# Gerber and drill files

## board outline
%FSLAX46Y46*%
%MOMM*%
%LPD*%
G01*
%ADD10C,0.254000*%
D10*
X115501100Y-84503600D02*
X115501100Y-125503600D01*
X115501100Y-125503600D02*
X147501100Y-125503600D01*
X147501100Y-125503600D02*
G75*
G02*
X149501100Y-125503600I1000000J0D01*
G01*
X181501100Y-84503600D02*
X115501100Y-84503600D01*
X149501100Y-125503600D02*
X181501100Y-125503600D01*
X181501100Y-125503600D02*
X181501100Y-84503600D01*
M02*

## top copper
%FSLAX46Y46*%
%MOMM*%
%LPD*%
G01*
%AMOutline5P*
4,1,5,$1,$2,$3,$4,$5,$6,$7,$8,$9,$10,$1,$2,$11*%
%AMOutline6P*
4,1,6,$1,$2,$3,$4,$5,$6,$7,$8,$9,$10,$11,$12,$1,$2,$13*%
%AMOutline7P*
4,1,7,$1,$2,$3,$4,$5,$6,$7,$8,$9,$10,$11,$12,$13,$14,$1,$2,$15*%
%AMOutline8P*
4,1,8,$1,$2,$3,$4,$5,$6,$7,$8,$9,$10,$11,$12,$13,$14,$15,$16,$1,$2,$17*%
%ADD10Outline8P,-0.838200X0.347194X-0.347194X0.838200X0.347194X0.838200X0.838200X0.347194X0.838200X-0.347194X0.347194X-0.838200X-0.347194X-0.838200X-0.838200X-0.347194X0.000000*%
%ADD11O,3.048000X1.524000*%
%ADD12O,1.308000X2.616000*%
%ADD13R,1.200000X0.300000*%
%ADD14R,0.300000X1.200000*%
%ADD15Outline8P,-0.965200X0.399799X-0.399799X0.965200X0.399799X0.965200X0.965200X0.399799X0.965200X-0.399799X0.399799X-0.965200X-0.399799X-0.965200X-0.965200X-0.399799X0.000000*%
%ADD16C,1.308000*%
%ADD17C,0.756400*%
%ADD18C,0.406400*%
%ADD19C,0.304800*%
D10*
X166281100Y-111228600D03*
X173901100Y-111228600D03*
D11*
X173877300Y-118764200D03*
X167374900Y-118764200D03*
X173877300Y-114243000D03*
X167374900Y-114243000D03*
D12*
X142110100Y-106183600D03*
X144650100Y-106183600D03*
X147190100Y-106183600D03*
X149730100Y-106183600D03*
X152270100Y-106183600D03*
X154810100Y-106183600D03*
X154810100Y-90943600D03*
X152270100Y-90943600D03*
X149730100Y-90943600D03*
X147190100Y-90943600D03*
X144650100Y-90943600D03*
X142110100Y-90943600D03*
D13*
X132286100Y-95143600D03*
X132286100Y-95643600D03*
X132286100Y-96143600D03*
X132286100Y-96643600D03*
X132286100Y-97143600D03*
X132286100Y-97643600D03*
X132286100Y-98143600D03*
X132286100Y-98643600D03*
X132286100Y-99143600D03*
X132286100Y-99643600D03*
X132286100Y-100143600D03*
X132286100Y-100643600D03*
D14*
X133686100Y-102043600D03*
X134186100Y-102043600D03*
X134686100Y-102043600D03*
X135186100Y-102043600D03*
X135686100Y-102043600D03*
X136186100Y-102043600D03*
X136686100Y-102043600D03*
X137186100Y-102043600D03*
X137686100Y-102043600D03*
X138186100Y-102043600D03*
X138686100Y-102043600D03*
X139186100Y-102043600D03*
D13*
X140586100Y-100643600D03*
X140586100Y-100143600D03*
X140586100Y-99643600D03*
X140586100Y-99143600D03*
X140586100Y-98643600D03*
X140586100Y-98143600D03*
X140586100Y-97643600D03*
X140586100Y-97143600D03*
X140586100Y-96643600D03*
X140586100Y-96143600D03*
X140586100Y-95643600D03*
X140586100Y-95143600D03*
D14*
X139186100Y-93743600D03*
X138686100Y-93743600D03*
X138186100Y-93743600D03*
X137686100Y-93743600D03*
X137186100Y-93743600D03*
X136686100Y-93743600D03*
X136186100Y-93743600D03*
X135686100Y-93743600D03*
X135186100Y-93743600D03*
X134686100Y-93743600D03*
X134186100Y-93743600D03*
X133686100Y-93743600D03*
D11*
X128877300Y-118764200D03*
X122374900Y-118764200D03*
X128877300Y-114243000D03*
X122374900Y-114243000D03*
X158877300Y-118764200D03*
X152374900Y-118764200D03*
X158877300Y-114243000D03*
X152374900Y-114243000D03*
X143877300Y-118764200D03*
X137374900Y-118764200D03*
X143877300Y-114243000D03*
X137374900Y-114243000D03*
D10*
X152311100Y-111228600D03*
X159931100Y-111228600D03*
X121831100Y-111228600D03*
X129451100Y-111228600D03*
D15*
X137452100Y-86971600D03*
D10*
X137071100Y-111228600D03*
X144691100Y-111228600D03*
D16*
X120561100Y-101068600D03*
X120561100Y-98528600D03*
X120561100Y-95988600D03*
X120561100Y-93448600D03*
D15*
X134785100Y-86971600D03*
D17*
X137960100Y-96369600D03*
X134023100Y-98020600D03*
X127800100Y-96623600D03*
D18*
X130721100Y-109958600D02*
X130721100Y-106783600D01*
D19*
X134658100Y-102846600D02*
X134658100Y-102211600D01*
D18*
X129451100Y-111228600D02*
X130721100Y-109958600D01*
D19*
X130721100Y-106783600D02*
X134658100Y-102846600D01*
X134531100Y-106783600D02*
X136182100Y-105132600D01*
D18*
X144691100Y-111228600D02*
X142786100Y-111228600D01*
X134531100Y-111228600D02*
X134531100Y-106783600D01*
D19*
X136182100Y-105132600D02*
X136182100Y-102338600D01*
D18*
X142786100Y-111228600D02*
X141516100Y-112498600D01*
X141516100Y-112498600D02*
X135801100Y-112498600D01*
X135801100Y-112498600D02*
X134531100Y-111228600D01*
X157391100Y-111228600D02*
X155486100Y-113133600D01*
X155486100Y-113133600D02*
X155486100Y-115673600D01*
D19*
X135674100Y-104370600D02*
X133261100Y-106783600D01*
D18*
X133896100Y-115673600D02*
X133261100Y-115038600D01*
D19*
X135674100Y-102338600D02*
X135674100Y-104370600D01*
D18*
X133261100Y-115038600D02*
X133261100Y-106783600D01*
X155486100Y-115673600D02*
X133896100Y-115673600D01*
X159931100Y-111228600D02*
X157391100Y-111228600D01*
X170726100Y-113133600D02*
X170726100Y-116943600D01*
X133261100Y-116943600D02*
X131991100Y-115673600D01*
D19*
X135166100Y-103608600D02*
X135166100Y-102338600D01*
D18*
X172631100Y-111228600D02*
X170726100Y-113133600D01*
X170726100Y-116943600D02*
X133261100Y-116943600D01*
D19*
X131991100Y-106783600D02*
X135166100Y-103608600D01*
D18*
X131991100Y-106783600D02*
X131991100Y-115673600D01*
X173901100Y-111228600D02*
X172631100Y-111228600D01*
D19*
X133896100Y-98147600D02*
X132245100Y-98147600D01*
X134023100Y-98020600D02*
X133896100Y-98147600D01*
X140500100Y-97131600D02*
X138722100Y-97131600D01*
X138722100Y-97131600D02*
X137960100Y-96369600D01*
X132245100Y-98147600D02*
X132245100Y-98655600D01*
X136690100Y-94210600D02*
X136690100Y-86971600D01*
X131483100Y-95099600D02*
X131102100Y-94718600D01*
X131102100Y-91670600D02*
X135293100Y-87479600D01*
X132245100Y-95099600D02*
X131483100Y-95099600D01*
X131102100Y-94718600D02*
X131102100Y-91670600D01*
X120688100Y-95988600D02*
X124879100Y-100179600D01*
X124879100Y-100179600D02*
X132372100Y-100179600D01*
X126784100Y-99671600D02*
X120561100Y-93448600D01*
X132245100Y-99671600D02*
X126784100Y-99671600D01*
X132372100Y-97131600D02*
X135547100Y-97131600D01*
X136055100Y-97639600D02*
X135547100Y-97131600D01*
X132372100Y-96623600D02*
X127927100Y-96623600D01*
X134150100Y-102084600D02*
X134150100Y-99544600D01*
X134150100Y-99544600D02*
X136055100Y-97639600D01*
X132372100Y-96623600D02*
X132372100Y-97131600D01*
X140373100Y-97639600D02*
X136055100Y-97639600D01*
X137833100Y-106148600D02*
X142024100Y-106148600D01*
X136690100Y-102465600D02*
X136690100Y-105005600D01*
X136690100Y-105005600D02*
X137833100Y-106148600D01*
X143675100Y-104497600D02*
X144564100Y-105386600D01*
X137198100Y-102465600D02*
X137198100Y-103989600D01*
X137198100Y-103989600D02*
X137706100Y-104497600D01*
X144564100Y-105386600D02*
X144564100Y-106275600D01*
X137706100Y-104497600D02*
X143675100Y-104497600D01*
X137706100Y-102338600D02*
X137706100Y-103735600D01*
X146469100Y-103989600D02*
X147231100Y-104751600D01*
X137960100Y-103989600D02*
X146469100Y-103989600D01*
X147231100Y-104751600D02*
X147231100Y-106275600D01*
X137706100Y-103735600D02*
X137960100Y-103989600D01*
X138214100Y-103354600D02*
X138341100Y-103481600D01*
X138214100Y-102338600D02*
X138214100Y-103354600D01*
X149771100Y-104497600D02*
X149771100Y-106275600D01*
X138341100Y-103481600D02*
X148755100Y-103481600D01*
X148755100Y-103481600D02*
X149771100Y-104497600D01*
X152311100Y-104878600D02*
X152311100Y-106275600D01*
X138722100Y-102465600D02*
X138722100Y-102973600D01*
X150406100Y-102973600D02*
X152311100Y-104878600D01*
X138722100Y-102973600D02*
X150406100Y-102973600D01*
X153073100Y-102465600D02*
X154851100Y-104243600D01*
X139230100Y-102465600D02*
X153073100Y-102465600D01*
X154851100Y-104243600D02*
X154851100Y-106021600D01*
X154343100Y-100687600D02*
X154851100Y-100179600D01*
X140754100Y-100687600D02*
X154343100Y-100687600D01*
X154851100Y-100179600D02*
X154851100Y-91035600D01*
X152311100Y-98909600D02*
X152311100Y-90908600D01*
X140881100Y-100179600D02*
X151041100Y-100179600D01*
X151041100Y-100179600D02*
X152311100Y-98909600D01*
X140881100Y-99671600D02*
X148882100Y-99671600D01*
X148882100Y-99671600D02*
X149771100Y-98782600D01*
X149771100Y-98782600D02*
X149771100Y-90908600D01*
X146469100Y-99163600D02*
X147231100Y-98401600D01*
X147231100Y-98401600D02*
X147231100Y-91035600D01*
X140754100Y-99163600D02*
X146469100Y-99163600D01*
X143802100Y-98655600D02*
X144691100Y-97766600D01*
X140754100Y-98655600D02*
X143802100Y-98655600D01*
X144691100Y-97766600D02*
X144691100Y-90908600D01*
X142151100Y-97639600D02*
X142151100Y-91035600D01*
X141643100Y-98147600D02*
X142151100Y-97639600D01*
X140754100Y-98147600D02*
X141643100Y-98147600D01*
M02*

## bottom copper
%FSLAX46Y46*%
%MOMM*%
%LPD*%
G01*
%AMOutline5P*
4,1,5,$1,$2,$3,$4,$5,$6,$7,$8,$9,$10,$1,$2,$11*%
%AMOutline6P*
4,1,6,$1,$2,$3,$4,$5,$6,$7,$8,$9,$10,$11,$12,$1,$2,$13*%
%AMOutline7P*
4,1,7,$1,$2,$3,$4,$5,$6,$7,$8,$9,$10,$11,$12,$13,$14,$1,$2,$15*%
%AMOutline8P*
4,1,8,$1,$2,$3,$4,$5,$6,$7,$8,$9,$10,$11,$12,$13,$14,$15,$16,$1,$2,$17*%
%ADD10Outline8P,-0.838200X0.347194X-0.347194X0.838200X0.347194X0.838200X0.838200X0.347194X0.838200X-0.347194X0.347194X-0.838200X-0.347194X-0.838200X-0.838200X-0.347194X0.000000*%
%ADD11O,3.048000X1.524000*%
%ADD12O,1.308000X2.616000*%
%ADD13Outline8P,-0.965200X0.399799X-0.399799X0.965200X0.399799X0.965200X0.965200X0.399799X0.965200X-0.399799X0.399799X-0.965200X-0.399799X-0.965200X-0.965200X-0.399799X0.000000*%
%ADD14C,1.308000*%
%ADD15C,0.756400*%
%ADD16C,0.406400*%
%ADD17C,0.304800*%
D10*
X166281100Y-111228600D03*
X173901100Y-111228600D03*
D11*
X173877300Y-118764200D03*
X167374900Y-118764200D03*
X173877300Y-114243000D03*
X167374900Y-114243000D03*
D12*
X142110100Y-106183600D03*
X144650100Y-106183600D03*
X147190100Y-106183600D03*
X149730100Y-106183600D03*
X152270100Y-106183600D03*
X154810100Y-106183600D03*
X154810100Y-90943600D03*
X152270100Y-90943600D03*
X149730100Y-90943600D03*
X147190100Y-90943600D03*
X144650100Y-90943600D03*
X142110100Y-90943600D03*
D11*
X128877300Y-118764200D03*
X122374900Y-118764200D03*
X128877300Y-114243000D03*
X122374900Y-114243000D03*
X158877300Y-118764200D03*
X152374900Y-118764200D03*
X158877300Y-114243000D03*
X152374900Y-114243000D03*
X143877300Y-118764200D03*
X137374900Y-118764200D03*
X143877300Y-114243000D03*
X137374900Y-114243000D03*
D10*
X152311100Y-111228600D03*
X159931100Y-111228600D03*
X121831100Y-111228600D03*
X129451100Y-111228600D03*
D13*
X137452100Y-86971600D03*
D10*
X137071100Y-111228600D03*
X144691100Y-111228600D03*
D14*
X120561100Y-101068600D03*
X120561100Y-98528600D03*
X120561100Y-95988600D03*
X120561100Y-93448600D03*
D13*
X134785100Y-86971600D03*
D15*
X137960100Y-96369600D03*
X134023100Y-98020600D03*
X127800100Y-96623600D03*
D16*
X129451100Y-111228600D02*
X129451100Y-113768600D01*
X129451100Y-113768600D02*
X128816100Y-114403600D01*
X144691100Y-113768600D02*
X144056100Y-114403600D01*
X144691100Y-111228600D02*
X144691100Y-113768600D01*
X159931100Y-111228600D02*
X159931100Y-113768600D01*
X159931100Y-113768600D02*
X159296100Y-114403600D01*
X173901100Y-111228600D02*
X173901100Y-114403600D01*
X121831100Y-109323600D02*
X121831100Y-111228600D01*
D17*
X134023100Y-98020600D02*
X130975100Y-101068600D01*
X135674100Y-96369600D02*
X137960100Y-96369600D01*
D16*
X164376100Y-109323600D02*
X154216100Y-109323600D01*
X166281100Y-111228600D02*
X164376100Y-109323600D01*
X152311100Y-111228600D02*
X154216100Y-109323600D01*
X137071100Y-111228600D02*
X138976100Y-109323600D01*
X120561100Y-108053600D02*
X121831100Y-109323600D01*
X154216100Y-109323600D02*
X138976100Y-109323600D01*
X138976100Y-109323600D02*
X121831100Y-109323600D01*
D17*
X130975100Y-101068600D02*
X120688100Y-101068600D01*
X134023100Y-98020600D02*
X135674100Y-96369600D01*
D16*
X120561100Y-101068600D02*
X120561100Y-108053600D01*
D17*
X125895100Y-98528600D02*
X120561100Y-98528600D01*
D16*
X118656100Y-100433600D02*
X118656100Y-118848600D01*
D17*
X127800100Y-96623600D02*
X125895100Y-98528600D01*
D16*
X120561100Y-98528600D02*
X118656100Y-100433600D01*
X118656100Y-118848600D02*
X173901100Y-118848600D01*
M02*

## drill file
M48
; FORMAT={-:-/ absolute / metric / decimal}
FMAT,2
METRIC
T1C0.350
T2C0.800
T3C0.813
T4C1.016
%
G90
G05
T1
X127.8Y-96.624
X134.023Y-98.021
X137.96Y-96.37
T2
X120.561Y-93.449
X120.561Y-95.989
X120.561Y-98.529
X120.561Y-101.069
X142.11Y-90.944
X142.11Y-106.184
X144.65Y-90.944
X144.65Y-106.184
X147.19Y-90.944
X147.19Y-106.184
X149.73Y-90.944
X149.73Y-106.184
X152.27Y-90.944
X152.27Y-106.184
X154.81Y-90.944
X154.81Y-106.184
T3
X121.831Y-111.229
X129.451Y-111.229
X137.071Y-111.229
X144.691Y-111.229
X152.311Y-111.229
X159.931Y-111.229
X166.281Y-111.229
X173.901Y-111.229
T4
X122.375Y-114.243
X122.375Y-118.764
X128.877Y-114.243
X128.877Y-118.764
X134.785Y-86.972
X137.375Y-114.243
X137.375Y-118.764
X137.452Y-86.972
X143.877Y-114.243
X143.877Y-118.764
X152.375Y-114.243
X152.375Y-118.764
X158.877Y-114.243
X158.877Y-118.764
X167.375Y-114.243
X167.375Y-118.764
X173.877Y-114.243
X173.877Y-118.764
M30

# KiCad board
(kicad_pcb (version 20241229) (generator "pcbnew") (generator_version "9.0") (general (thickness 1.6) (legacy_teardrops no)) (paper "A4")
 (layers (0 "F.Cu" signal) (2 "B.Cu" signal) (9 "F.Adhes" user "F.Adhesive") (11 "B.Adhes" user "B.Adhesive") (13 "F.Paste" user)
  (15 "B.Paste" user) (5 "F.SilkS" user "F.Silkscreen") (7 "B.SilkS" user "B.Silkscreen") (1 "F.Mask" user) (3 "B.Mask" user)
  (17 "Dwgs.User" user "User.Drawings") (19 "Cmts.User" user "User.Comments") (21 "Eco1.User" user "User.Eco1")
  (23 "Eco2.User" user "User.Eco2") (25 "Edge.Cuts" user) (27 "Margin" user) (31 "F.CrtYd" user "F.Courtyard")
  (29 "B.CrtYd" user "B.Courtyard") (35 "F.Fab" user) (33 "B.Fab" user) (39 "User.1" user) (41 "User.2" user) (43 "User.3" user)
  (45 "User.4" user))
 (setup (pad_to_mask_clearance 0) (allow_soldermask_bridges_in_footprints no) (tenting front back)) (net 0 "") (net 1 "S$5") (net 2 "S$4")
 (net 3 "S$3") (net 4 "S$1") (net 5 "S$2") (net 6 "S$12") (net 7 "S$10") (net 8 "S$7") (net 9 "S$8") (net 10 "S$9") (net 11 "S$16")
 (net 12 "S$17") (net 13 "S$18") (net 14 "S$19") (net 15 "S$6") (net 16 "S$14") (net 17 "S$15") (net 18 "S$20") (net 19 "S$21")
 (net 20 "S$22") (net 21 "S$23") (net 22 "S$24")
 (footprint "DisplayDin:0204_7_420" (layer "F.Cu") (at 170.0911 111.2286)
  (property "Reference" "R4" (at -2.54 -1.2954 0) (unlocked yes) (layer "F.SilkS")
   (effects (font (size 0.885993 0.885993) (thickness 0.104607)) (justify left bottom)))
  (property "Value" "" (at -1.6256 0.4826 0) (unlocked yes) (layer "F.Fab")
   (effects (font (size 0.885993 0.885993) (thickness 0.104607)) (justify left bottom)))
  (pad "1" thru_hole roundrect (at -3.81 0) (size 1.6764 1.6764) (drill 0.8128) (layers "*.Cu" "*.Mask") (remove_unused_layers no)
   (roundrect_rratio 0.25) (chamfer_ratio 0.2928932188) (chamfer top_left top_right bottom_left bottom_right) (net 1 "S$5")
   (solder_mask_margin 0.1016) (thermal_bridge_angle 0))
  (pad "2" thru_hole roundrect (at 3.81 0) (size 1.6764 1.6764) (drill 0.8128) (layers "*.Cu" "*.Mask") (remove_unused_layers no)
   (roundrect_rratio 0.25) (chamfer_ratio 0.2928932188) (chamfer top_left top_right bottom_left bottom_right) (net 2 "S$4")
   (solder_mask_margin 0.1016) (thermal_bridge_angle 0)))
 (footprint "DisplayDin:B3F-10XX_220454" (layer "F.Cu") (at 170.6261 116.5036 180)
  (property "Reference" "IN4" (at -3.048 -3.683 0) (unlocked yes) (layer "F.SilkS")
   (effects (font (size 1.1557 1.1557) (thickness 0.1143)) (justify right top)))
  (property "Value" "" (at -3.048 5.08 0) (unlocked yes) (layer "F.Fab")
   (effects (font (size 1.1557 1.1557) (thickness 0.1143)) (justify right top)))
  (pad "1" thru_hole oval (at -3.2512 -2.2606 180) (size 3.048 1.524) (drill 1.016) (layers "*.Cu" "*.Mask") (remove_unused_layers no)
   (solder_mask_margin 0.1016) (thermal_bridge_angle 0))
  (pad "2" thru_hole oval (at 3.2512 -2.2606 180) (size 3.048 1.524) (drill 1.016) (layers "*.Cu" "*.Mask") (remove_unused_layers no)
   (solder_mask_margin 0.1016) (thermal_bridge_angle 0))
  (pad "3" thru_hole oval (at -3.2512 2.2606 180) (size 3.048 1.524) (drill 1.016) (layers "*.Cu" "*.Mask") (remove_unused_layers no)
   (solder_mask_margin 0.1016) (thermal_bridge_angle 0))
  (pad "4" thru_hole oval (at 3.2512 2.2606 180) (size 3.048 1.524) (drill 1.016) (layers "*.Cu" "*.Mask") (remove_unused_layers no)
   (solder_mask_margin 0.1016) (thermal_bridge_angle 0)))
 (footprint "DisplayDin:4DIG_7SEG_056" (layer "F.Cu") (at 143.1261 94.7536)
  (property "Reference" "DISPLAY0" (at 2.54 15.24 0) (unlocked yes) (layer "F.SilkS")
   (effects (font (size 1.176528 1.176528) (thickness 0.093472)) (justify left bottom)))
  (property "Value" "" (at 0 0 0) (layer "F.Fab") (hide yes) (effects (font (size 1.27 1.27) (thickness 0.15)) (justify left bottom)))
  (pad "1" thru_hole oval (at -1.016 11.43 90) (size 2.616 1.308) (drill 0.8) (layers "*.Cu" "*.Mask") (remove_unused_layers no)
   (solder_mask_margin 0.1016) (thermal_bridge_angle 0))
  (pad "2" thru_hole oval (at 1.524 11.43 90) (size 2.616 1.308) (drill 0.8) (layers "*.Cu" "*.Mask") (remove_unused_layers no)
   (solder_mask_margin 0.1016) (thermal_bridge_angle 0))
  (pad "3" thru_hole oval (at 4.064 11.43 90) (size 2.616 1.308) (drill 0.8) (layers "*.Cu" "*.Mask") (remove_unused_layers no)
   (solder_mask_margin 0.1016) (thermal_bridge_angle 0))
  (pad "4" thru_hole oval (at 6.604 11.43 90) (size 2.616 1.308) (drill 0.8) (layers "*.Cu" "*.Mask") (remove_unused_layers no)
   (solder_mask_margin 0.1016) (thermal_bridge_angle 0))
  (pad "5" thru_hole oval (at 9.144 11.43 90) (size 2.616 1.308) (drill 0.8) (layers "*.Cu" "*.Mask") (remove_unused_layers no)
   (solder_mask_margin 0.1016) (thermal_bridge_angle 0))
  (pad "6" thru_hole oval (at 11.684 11.43 90) (size 2.616 1.308) (drill 0.8) (layers "*.Cu" "*.Mask") (remove_unused_layers no)
   (solder_mask_margin 0.1016) (thermal_bridge_angle 0))
  (pad "9" thru_hole oval (at 11.684 -3.81 90) (size 2.616 1.308) (drill 0.8) (layers "*.Cu" "*.Mask") (remove_unused_layers no)
   (solder_mask_margin 0.1016) (thermal_bridge_angle 0))
  (pad "10" thru_hole oval (at 9.144 -3.81 270) (size 2.616 1.308) (drill 0.8) (layers "*.Cu" "*.Mask") (remove_unused_layers no)
   (solder_mask_margin 0.1016) (thermal_bridge_angle 0))
  (pad "11" thru_hole oval (at 6.604 -3.81 270) (size 2.616 1.308) (drill 0.8) (layers "*.Cu" "*.Mask") (remove_unused_layers no)
   (solder_mask_margin 0.1016) (thermal_bridge_angle 0))
  (pad "12" thru_hole oval (at 4.064 -3.81 270) (size 2.616 1.308) (drill 0.8) (layers "*.Cu" "*.Mask") (remove_unused_layers no)
   (solder_mask_margin 0.1016) (thermal_bridge_angle 0))
  (pad "13" thru_hole oval (at 1.524 -3.81 270) (size 2.616 1.308) (drill 0.8) (layers "*.Cu" "*.Mask") (remove_unused_layers no)
   (solder_mask_margin 0.1016) (thermal_bridge_angle 0))
  (pad "14" thru_hole oval (at -1.016 -3.81 270) (size 2.616 1.308) (drill 0.8) (layers "*.Cu" "*.Mask") (remove_unused_layers no)
   (solder_mask_margin 0.1016) (thermal_bridge_angle 0)))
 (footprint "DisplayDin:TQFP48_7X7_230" (layer "F.Cu") (at 136.4361 97.8936 -90)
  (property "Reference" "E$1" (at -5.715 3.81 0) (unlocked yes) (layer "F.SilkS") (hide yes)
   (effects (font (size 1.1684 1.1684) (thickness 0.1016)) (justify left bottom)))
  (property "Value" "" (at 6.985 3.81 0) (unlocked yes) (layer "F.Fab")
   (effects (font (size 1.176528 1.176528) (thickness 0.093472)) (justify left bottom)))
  (pad "1" smd rect (at -2.75 4.15 270) (size 0.3 1.2) (layers "F.Cu" "F.Mask" "F.Paste") (solder_mask_margin 0.1016)
   (solder_paste_margin 0) (thermal_bridge_angle 0))
  (pad "2" smd rect (at -2.25 4.15 270) (size 0.3 1.2) (layers "F.Cu" "F.Mask" "F.Paste") (solder_mask_margin 0.1016)
   (solder_paste_margin 0) (thermal_bridge_angle 0))
  (pad "3" smd rect (at -1.75 4.15 270) (size 0.3 1.2) (layers "F.Cu" "F.Mask" "F.Paste") (solder_mask_margin 0.1016)
   (solder_paste_margin 0) (thermal_bridge_angle 0))
  (pad "4" smd rect (at -1.25 4.15 270) (size 0.3 1.2) (layers "F.Cu" "F.Mask" "F.Paste") (solder_mask_margin 0.1016)
   (solder_paste_margin 0) (thermal_bridge_angle 0))
  (pad "5" smd rect (at -0.75 4.15 270) (size 0.3 1.2) (layers "F.Cu" "F.Mask" "F.Paste") (solder_mask_margin 0.1016)
   (solder_paste_margin 0) (thermal_bridge_angle 0))
  (pad "6" smd rect (at -0.25 4.15 270) (size 0.3 1.2) (layers "F.Cu" "F.Mask" "F.Paste") (solder_mask_margin 0.1016)
   (solder_paste_margin 0) (thermal_bridge_angle 0))
  (pad "7" smd rect (at 0.25 4.15 270) (size 0.3 1.2) (layers "F.Cu" "F.Mask" "F.Paste") (solder_mask_margin 0.1016) (solder_paste_margin 0)
   (thermal_bridge_angle 0))
  (pad "8" smd rect (at 0.75 4.15 270) (size 0.3 1.2) (layers "F.Cu" "F.Mask" "F.Paste") (solder_mask_margin 0.1016) (solder_paste_margin 0)
   (thermal_bridge_angle 0))
  (pad "9" smd rect (at 1.25 4.15 270) (size 0.3 1.2) (layers "F.Cu" "F.Mask" "F.Paste") (solder_mask_margin 0.1016) (solder_paste_margin 0)
   (thermal_bridge_angle 0))
  (pad "10" smd rect (at 1.75 4.15 270) (size 0.3 1.2) (layers "F.Cu" "F.Mask" "F.Paste") (solder_mask_margin 0.1016)
   (solder_paste_margin 0) (thermal_bridge_angle 0))
  (pad "11" smd rect (at 2.25 4.15 270) (size 0.3 1.2) (layers "F.Cu" "F.Mask" "F.Paste") (solder_mask_margin 0.1016)
   (solder_paste_margin 0) (thermal_bridge_angle 0))
  (pad "12" smd rect (at 2.75 4.15 270) (size 0.3 1.2) (layers "F.Cu" "F.Mask" "F.Paste") (solder_mask_margin 0.1016)
   (solder_paste_margin 0) (thermal_bridge_angle 0))
  (pad "13" smd rect (at 4.15 2.75 270) (size 1.2 0.3) (layers "F.Cu" "F.Mask" "F.Paste") (solder_mask_margin 0.1016)
   (solder_paste_margin 0) (thermal_bridge_angle 0))
  (pad "14" smd rect (at 4.15 2.25 270) (size 1.2 0.3) (layers "F.Cu" "F.Mask" "F.Paste") (solder_mask_margin 0.1016)
   (solder_paste_margin 0) (thermal_bridge_angle 0))
  (pad "15" smd rect (at 4.15 1.75 270) (size 1.2 0.3) (layers "F.Cu" "F.Mask" "F.Paste") (solder_mask_margin 0.1016)
   (solder_paste_margin 0) (thermal_bridge_angle 0))
  (pad "16" smd rect (at 4.15 1.25 270) (size 1.2 0.3) (layers "F.Cu" "F.Mask" "F.Paste") (solder_mask_margin 0.1016)
   (solder_paste_margin 0) (thermal_bridge_angle 0))
  (pad "17" smd rect (at 4.15 0.75 270) (size 1.2 0.3) (layers "F.Cu" "F.Mask" "F.Paste") (solder_mask_margin 0.1016)
   (solder_paste_margin 0) (thermal_bridge_angle 0))
  (pad "18" smd rect (at 4.15 0.25 270) (size 1.2 0.3) (layers "F.Cu" "F.Mask" "F.Paste") (solder_mask_margin 0.1016)
   (solder_paste_margin 0) (thermal_bridge_angle 0))
  (pad "19" smd rect (at 4.15 -0.25 270) (size 1.2 0.3) (layers "F.Cu" "F.Mask" "F.Paste") (solder_mask_margin 0.1016)
   (solder_paste_margin 0) (thermal_bridge_angle 0))
  (pad "20" smd rect (at 4.15 -0.75 270) (size 1.2 0.3) (layers "F.Cu" "F.Mask" "F.Paste") (solder_mask_margin 0.1016)
   (solder_paste_margin 0) (thermal_bridge_angle 0))
  (pad "21" smd rect (at 4.15 -1.25 270) (size 1.2 0.3) (layers "F.Cu" "F.Mask" "F.Paste") (solder_mask_margin 0.1016)
   (solder_paste_margin 0) (thermal_bridge_angle 0))
  (pad "22" smd rect (at 4.15 -1.75 270) (size 1.2 0.3) (layers "F.Cu" "F.Mask" "F.Paste") (solder_mask_margin 0.1016)
   (solder_paste_margin 0) (thermal_bridge_angle 0))
  (pad "23" smd rect (at 4.15 -2.25 270) (size 1.2 0.3) (layers "F.Cu" "F.Mask" "F.Paste") (solder_mask_margin 0.1016)
   (solder_paste_margin 0) (thermal_bridge_angle 0))
  (pad "24" smd rect (at 4.15 -2.75 270) (size 1.2 0.3) (layers "F.Cu" "F.Mask" "F.Paste") (solder_mask_margin 0.1016)
   (solder_paste_margin 0) (thermal_bridge_angle 0))
  (pad "25" smd rect (at 2.75 -4.15 270) (size 0.3 1.2) (layers "F.Cu" "F.Mask" "F.Paste") (solder_mask_margin 0.1016)
   (solder_paste_margin 0) (thermal_bridge_angle 0))
  (pad "26" smd rect (at 2.25 -4.15 270) (size 0.3 1.2) (layers "F.Cu" "F.Mask" "F.Paste") (solder_mask_margin 0.1016)
   (solder_paste_margin 0) (thermal_bridge_angle 0))
  (pad "27" smd rect (at 1.75 -4.15 270) (size 0.3 1.2) (layers "F.Cu" "F.Mask" "F.Paste") (solder_mask_margin 0.1016)
   (solder_paste_margin 0) (thermal_bridge_angle 0))
  (pad "28" smd rect (at 1.25 -4.15 270) (size 0.3 1.2) (layers "F.Cu" "F.Mask" "F.Paste") (solder_mask_margin 0.1016)
   (solder_paste_margin 0) (thermal_bridge_angle 0))
  (pad "29" smd rect (at 0.75 -4.15 270) (size 0.3 1.2) (layers "F.Cu" "F.Mask" "F.Paste") (solder_mask_margin 0.1016)
   (solder_paste_margin 0) (thermal_bridge_angle 0))
  (pad "30" smd rect (at 0.25 -4.15 270) (size 0.3 1.2) (layers "F.Cu" "F.Mask" "F.Paste") (solder_mask_margin 0.1016)
   (solder_paste_margin 0) (thermal_bridge_angle 0))
  (pad "31" smd rect (at -0.25 -4.15 270) (size 0.3 1.2) (layers "F.Cu" "F.Mask" "F.Paste") (solder_mask_margin 0.1016)
   (solder_paste_margin 0) (thermal_bridge_angle 0))
  (pad "32" smd rect (at -0.75 -4.15 270) (size 0.3 1.2) (layers "F.Cu" "F.Mask" "F.Paste") (solder_mask_margin 0.1016)
   (solder_paste_margin 0) (thermal_bridge_angle 0))
  (pad "33" smd rect (at -1.25 -4.15 270) (size 0.3 1.2) (layers "F.Cu" "F.Mask" "F.Paste") (solder_mask_margin 0.1016)
   (solder_paste_margin 0) (thermal_bridge_angle 0))
  (pad "34" smd rect (at -1.75 -4.15 270) (size 0.3 1.2) (layers "F.Cu" "F.Mask" "F.Paste") (solder_mask_margin 0.1016)
   (solder_paste_margin 0) (thermal_bridge_angle 0))
  (pad "35" smd rect (at -2.25 -4.15 270) (size 0.3 1.2) (layers "F.Cu" "F.Mask" "F.Paste") (solder_mask_margin 0.1016)
   (solder_paste_margin 0) (thermal_bridge_angle 0))
  (pad "36" smd rect (at -2.75 -4.15 270) (size 0.3 1.2) (layers "F.Cu" "F.Mask" "F.Paste") (solder_mask_margin 0.1016)
   (solder_paste_margin 0) (thermal_bridge_angle 0))
  (pad "37" smd rect (at -4.15 -2.75 270) (size 1.2 0.3) (layers "F.Cu" "F.Mask" "F.Paste") (solder_mask_margin 0.1016)
   (solder_paste_margin 0) (thermal_bridge_angle 0))
  (pad "38" smd rect (at -4.15 -2.25 270) (size 1.2 0.3) (layers "F.Cu" "F.Mask" "F.Paste") (solder_mask_margin 0.1016)
   (solder_paste_margin 0) (thermal_bridge_angle 0))
  (pad "39" smd rect (at -4.15 -1.75 270) (size 1.2 0.3) (layers "F.Cu" "F.Mask" "F.Paste") (solder_mask_margin 0.1016)
   (solder_paste_margin 0) (thermal_bridge_angle 0))
  (pad "40" smd rect (at -4.15 -1.25 270) (size 1.2 0.3) (layers "F.Cu" "F.Mask" "F.Paste") (solder_mask_margin 0.1016)
   (solder_paste_margin 0) (thermal_bridge_angle 0))
  (pad "41" smd rect (at -4.15 -0.75 270) (size 1.2 0.3) (layers "F.Cu" "F.Mask" "F.Paste") (solder_mask_margin 0.1016)
   (solder_paste_margin 0) (thermal_bridge_angle 0))
  (pad "42" smd rect (at -4.15 -0.25 270) (size 1.2 0.3) (layers "F.Cu" "F.Mask" "F.Paste") (solder_mask_margin 0.1016)
   (solder_paste_margin 0) (thermal_bridge_angle 0))
  (pad "43" smd rect (at -4.15 0.25 270) (size 1.2 0.3) (layers "F.Cu" "F.Mask" "F.Paste") (solder_mask_margin 0.1016)
   (solder_paste_margin 0) (thermal_bridge_angle 0))
  (pad "44" smd rect (at -4.15 0.75 270) (size 1.2 0.3) (layers "F.Cu" "F.Mask" "F.Paste") (solder_mask_margin 0.1016)
   (solder_paste_margin 0) (thermal_bridge_angle 0))
  (pad "45" smd rect (at -4.15 1.25 270) (size 1.2 0.3) (layers "F.Cu" "F.Mask" "F.Paste") (solder_mask_margin 0.1016)
   (solder_paste_margin 0) (thermal_bridge_angle 0))
  (pad "46" smd rect (at -4.15 1.75 270) (size 1.2 0.3) (layers "F.Cu" "F.Mask" "F.Paste") (solder_mask_margin 0.1016)
   (solder_paste_margin 0) (thermal_bridge_angle 0))
  (pad "47" smd rect (at -4.15 2.25 270) (size 1.2 0.3) (layers "F.Cu" "F.Mask" "F.Paste") (solder_mask_margin 0.1016)
   (solder_paste_margin 0) (thermal_bridge_angle 0))
  (pad "48" smd rect (at -4.15 2.75 270) (size 1.2 0.3) (layers "F.Cu" "F.Mask" "F.Paste") (solder_mask_margin 0.1016)
   (solder_paste_margin 0) (thermal_bridge_angle 0)))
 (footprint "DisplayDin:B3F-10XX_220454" (layer "F.Cu") (at 125.6261 116.5036 180)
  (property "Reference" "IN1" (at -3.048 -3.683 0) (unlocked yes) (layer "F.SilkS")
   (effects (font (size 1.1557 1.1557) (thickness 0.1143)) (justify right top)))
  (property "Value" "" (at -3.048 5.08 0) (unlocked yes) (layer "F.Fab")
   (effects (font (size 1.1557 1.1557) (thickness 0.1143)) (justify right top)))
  (pad "1" thru_hole oval (at -3.2512 -2.2606 180) (size 3.048 1.524) (drill 1.016) (layers "*.Cu" "*.Mask") (remove_unused_layers no)
   (solder_mask_margin 0.1016) (thermal_bridge_angle 0))
  (pad "2" thru_hole oval (at 3.2512 -2.2606 180) (size 3.048 1.524) (drill 1.016) (layers "*.Cu" "*.Mask") (remove_unused_layers no)
   (solder_mask_margin 0.1016) (thermal_bridge_angle 0))
  (pad "3" thru_hole oval (at -3.2512 2.2606 180) (size 3.048 1.524) (drill 1.016) (layers "*.Cu" "*.Mask") (remove_unused_layers no)
   (solder_mask_margin 0.1016) (thermal_bridge_angle 0))
  (pad "4" thru_hole oval (at 3.2512 2.2606 180) (size 3.048 1.524) (drill 1.016) (layers "*.Cu" "*.Mask") (remove_unused_layers no)
   (solder_mask_margin 0.1016) (thermal_bridge_angle 0)))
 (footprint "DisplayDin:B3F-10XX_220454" (layer "F.Cu") (at 155.6261 116.5036 180)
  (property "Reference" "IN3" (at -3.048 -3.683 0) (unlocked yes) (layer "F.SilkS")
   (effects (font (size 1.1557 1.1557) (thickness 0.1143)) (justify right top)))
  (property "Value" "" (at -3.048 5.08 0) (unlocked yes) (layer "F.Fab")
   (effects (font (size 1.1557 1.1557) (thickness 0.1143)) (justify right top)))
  (pad "1" thru_hole oval (at -3.2512 -2.2606 180) (size 3.048 1.524) (drill 1.016) (layers "*.Cu" "*.Mask") (remove_unused_layers no)
   (solder_mask_margin 0.1016) (thermal_bridge_angle 0))
  (pad "2" thru_hole oval (at 3.2512 -2.2606 180) (size 3.048 1.524) (drill 1.016) (layers "*.Cu" "*.Mask") (remove_unused_layers no)
   (solder_mask_margin 0.1016) (thermal_bridge_angle 0))
  (pad "3" thru_hole oval (at -3.2512 2.2606 180) (size 3.048 1.524) (drill 1.016) (layers "*.Cu" "*.Mask") (remove_unused_layers no)
   (solder_mask_margin 0.1016) (thermal_bridge_angle 0))
  (pad "4" thru_hole oval (at 3.2512 2.2606 180) (size 3.048 1.524) (drill 1.016) (layers "*.Cu" "*.Mask") (remove_unused_layers no)
   (solder_mask_margin 0.1016) (thermal_bridge_angle 0)))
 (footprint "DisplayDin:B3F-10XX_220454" (layer "F.Cu") (at 140.6261 116.5036 180)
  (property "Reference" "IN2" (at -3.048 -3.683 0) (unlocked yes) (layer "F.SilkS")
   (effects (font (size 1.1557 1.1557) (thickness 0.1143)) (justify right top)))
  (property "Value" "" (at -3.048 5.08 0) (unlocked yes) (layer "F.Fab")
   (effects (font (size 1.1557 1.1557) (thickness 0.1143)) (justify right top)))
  (pad "1" thru_hole oval (at -3.2512 -2.2606 180) (size 3.048 1.524) (drill 1.016) (layers "*.Cu" "*.Mask") (remove_unused_layers no)
   (solder_mask_margin 0.1016) (thermal_bridge_angle 0))
  (pad "2" thru_hole oval (at 3.2512 -2.2606 180) (size 3.048 1.524) (drill 1.016) (layers "*.Cu" "*.Mask") (remove_unused_layers no)
   (solder_mask_margin 0.1016) (thermal_bridge_angle 0))
  (pad "3" thru_hole oval (at -3.2512 2.2606 180) (size 3.048 1.524) (drill 1.016) (layers "*.Cu" "*.Mask") (remove_unused_layers no)
   (solder_mask_margin 0.1016) (thermal_bridge_angle 0))
  (pad "4" thru_hole oval (at 3.2512 2.2606 180) (size 3.048 1.524) (drill 1.016) (layers "*.Cu" "*.Mask") (remove_unused_layers no)
   (solder_mask_margin 0.1016) (thermal_bridge_angle 0)))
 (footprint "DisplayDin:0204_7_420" (layer "F.Cu") (at 156.1211 111.2286)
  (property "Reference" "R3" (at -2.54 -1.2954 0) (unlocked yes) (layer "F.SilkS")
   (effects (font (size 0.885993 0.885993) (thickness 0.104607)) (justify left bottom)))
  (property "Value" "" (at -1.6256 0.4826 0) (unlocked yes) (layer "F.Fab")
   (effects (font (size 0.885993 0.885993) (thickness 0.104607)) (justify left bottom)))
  (pad "1" thru_hole roundrect (at -3.81 0) (size 1.6764 1.6764) (drill 0.8128) (layers "*.Cu" "*.Mask") (remove_unused_layers no)
   (roundrect_rratio 0.25) (chamfer_ratio 0.2928932188) (chamfer top_left top_right bottom_left bottom_right) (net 1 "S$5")
   (solder_mask_margin 0.1016) (thermal_bridge_angle 0))
  (pad "2" thru_hole roundrect (at 3.81 0) (size 1.6764 1.6764) (drill 0.8128) (layers "*.Cu" "*.Mask") (remove_unused_layers no)
   (roundrect_rratio 0.25) (chamfer_ratio 0.2928932188) (chamfer top_left top_right bottom_left bottom_right) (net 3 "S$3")
   (solder_mask_margin 0.1016) (thermal_bridge_angle 0)))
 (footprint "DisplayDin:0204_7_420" (layer "F.Cu") (at 125.6411 111.2286)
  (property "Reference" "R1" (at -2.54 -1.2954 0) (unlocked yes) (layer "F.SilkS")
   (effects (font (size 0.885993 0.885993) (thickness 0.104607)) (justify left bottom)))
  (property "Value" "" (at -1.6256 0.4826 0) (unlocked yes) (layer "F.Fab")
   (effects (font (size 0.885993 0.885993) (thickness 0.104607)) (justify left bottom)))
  (pad "1" thru_hole roundrect (at -3.81 0) (size 1.6764 1.6764) (drill 0.8128) (layers "*.Cu" "*.Mask") (remove_unused_layers no)
   (roundrect_rratio 0.25) (chamfer_ratio 0.2928932188) (chamfer top_left top_right bottom_left bottom_right) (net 1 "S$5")
   (solder_mask_margin 0.1016) (thermal_bridge_angle 0))
  (pad "2" thru_hole roundrect (at 3.81 0) (size 1.6764 1.6764) (drill 0.8128) (layers "*.Cu" "*.Mask") (remove_unused_layers no)
   (roundrect_rratio 0.25) (chamfer_ratio 0.2928932188) (chamfer top_left top_right bottom_left bottom_right) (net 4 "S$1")
   (solder_mask_margin 0.1016) (thermal_bridge_angle 0)))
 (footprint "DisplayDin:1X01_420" (layer "F.Cu") (at 137.4521 86.9716)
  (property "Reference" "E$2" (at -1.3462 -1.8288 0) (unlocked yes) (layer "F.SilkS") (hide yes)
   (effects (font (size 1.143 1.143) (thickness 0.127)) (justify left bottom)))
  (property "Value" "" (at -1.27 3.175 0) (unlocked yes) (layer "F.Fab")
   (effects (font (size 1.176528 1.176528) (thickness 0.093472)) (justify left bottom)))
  (pad "1" thru_hole roundrect (at 0 0) (size 1.9304 1.9304) (drill 1.016) (layers "*.Cu" "*.Mask") (remove_unused_layers no)
   (roundrect_rratio 0.25) (chamfer_ratio 0.2928932188) (chamfer top_left top_right bottom_left bottom_right) (solder_mask_margin 0.1016)
   (thermal_bridge_angle 0)))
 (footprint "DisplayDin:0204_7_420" (layer "F.Cu") (at 140.8811 111.2286)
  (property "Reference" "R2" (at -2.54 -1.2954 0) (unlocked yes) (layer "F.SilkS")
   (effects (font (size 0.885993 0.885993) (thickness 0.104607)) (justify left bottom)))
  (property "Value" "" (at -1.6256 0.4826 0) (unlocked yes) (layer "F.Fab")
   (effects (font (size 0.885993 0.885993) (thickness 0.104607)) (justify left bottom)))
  (pad "1" thru_hole roundrect (at -3.81 0) (size 1.6764 1.6764) (drill 0.8128) (layers "*.Cu" "*.Mask") (remove_unused_layers no)
   (roundrect_rratio 0.25) (chamfer_ratio 0.2928932188) (chamfer top_left top_right bottom_left bottom_right) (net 1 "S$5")
   (solder_mask_margin 0.1016) (thermal_bridge_angle 0))
  (pad "2" thru_hole roundrect (at 3.81 0) (size 1.6764 1.6764) (drill 0.8128) (layers "*.Cu" "*.Mask") (remove_unused_layers no)
   (roundrect_rratio 0.25) (chamfer_ratio 0.2928932188) (chamfer top_left top_right bottom_left bottom_right) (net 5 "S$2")
   (solder_mask_margin 0.1016) (thermal_bridge_angle 0)))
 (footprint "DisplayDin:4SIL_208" (layer "F.Cu") (at 120.5611 97.2586 90)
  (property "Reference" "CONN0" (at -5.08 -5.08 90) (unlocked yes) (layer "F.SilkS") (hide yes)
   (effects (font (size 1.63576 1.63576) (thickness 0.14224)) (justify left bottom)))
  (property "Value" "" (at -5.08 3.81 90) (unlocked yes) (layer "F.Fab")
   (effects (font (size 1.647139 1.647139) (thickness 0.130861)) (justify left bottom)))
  (pad "1" thru_hole circle (at -3.81 0 90) (size 1.308 1.308) (drill 0.8) (layers "*.Cu" "*.Mask") (remove_unused_layers no) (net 1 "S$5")
   (solder_mask_margin 0.1016) (thermal_bridge_angle 0))
  (pad "2" thru_hole circle (at -1.27 0 90) (size 1.308 1.308) (drill 0.8) (layers "*.Cu" "*.Mask") (remove_unused_layers no) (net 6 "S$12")
   (solder_mask_margin 0.1016) (thermal_bridge_angle 0))
  (pad "3" thru_hole circle (at 1.27 0 90) (size 1.308 1.308) (drill 0.8) (layers "*.Cu" "*.Mask") (remove_unused_layers no)
   (solder_mask_margin 0.1016) (thermal_bridge_angle 0))
  (pad "4" thru_hole circle (at 3.81 0 90) (size 1.308 1.308) (drill 0.8) (layers "*.Cu" "*.Mask") (remove_unused_layers no) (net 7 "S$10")
   (solder_mask_margin 0.1016) (thermal_bridge_angle 0)))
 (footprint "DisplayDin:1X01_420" (layer "F.Cu") (at 134.7851 86.9716)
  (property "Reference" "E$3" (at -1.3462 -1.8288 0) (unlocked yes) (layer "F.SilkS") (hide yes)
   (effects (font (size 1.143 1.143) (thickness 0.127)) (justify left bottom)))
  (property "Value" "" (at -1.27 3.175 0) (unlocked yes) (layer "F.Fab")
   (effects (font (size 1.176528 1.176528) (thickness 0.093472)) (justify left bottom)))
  (pad "1" thru_hole roundrect (at 0 0) (size 1.9304 1.9304) (drill 1.016) (layers "*.Cu" "*.Mask") (remove_unused_layers no)
   (roundrect_rratio 0.25) (chamfer_ratio 0.2928932188) (chamfer top_left top_right bottom_left bottom_right) (solder_mask_margin 0.1016)
   (thermal_bridge_angle 0)))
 (gr_line (start 115.5011 84.5036) (end 115.5011 125.5036) (stroke (width 0.254) (type solid)) (layer "Edge.Cuts"))
 (gr_line (start 115.5011 125.5036) (end 147.5011 125.5036) (stroke (width 0.254) (type solid)) (layer "Edge.Cuts"))
 (gr_arc (start 147.5011 125.5036) (mid 148.5011 124.5036) (end 149.5011 125.5036) (stroke (width 0.254) (type solid)) (layer "Edge.Cuts"))
 (gr_line (start 181.5011 84.5036) (end 115.5011 84.5036) (stroke (width 0.254) (type solid)) (layer "Edge.Cuts"))
 (gr_line (start 149.5011 125.5036) (end 181.5011 125.5036) (stroke (width 0.254) (type solid)) (layer "Edge.Cuts"))
 (gr_line (start 181.5011 125.5036) (end 181.5011 84.5036) (stroke (width 0.254) (type solid)) (layer "Edge.Cuts"))
 (segment (start 130.7211 109.9586) (end 130.7211 106.7836) (width 0.4064) (layer "F.Cu") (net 4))
 (segment (start 134.6581 102.8466) (end 134.6581 102.2116) (width 0.3048) (layer "F.Cu") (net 4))
 (segment (start 129.4511 111.2286) (end 130.7211 109.9586) (width 0.4064) (layer "F.Cu") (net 4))
 (segment (start 130.7211 106.7836) (end 134.6581 102.8466) (width 0.3048) (layer "F.Cu") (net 4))
 (segment (start 129.4511 111.2286) (end 129.4511 113.7686) (width 0.4064) (layer "B.Cu") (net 4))
 (segment (start 129.4511 113.7686) (end 128.8161 114.4036) (width 0.4064) (layer "B.Cu") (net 4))
 (segment (start 134.5311 106.7836) (end 136.1821 105.1326) (width 0.3048) (layer "F.Cu") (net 5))
 (segment (start 144.6911 111.2286) (end 142.7861 111.2286) (width 0.4064) (layer "F.Cu") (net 5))
 (segment (start 134.5311 111.2286) (end 134.5311 106.7836) (width 0.4064) (layer "F.Cu") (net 5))
 (segment (start 136.1821 105.1326) (end 136.1821 102.3386) (width 0.3048) (layer "F.Cu") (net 5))
 (segment (start 142.7861 111.2286) (end 141.5161 112.4986) (width 0.4064) (layer "F.Cu") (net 5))
 (segment (start 141.5161 112.4986) (end 135.8011 112.4986) (width 0.4064) (layer "F.Cu") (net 5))
 (segment (start 135.8011 112.4986) (end 134.5311 111.2286) (width 0.4064) (layer "F.Cu") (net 5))
 (segment (start 144.6911 113.7686) (end 144.0561 114.4036) (width 0.4064) (layer "B.Cu") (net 5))
 (segment (start 144.6911 111.2286) (end 144.6911 113.7686) (width 0.4064) (layer "B.Cu") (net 5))
 (segment (start 157.3911 111.2286) (end 155.4861 113.1336) (width 0.4064) (layer "F.Cu") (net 3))
 (segment (start 155.4861 113.1336) (end 155.4861 115.6736) (width 0.4064) (layer "F.Cu") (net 3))
 (segment (start 135.6741 104.3706) (end 133.2611 106.7836) (width 0.3048) (layer "F.Cu") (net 3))
 (segment (start 133.8961 115.6736) (end 133.2611 115.0386) (width 0.4064) (layer "F.Cu") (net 3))
 (segment (start 135.6741 102.3386) (end 135.6741 104.3706) (width 0.3048) (layer "F.Cu") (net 3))
 (segment (start 133.2611 115.0386) (end 133.2611 106.7836) (width 0.4064) (layer "F.Cu") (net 3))
 (segment (start 155.4861 115.6736) (end 133.8961 115.6736) (width 0.4064) (layer "F.Cu") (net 3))
 (segment (start 159.9311 111.2286) (end 157.3911 111.2286) (width 0.4064) (layer "F.Cu") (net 3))
 (segment (start 159.9311 111.2286) (end 159.9311 113.7686) (width 0.4064) (layer "B.Cu") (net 3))
 (segment (start 159.9311 113.7686) (end 159.2961 114.4036) (width 0.4064) (layer "B.Cu") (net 3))
 (segment (start 170.7261 113.1336) (end 170.7261 116.9436) (width 0.4064) (layer "F.Cu") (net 2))
 (segment (start 133.2611 116.9436) (end 131.9911 115.6736) (width 0.4064) (layer "F.Cu") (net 2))
 (segment (start 135.1661 103.6086) (end 135.1661 102.3386) (width 0.3048) (layer "F.Cu") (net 2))
 (segment (start 172.6311 111.2286) (end 170.7261 113.1336) (width 0.4064) (layer "F.Cu") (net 2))
 (segment (start 170.7261 116.9436) (end 133.2611 116.9436) (width 0.4064) (layer "F.Cu") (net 2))
 (segment (start 131.9911 106.7836) (end 135.1661 103.6086) (width 0.3048) (layer "F.Cu") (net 2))
 (segment (start 131.9911 106.7836) (end 131.9911 115.6736) (width 0.4064) (layer "F.Cu") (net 2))
 (segment (start 173.9011 111.2286) (end 172.6311 111.2286) (width 0.4064) (layer "F.Cu") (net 2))
 (segment (start 173.9011 111.2286) (end 173.9011 114.4036) (width 0.4064) (layer "B.Cu") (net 2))
 (segment (start 133.8961 98.1476) (end 132.2451 98.1476) (width 0.3048) (layer "F.Cu") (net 1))
 (segment (start 134.0231 98.0206) (end 133.8961 98.1476) (width 0.3048) (layer "F.Cu") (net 1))
 (segment (start 140.5001 97.1316) (end 138.7221 97.1316) (width 0.3048) (layer "F.Cu") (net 1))
 (segment (start 138.7221 97.1316) (end 137.9601 96.3696) (width 0.3048) (layer "F.Cu") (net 1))
 (segment (start 132.2451 98.1476) (end 132.2451 98.6556) (width 0.3048) (layer "F.Cu") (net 1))
 (via (at 137.9601 96.3696) (size 0.7564) (drill 0.35) (layers "F.Cu" "B.Cu") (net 1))
 (via (at 134.0231 98.0206) (size 0.7564) (drill 0.35) (layers "F.Cu" "B.Cu") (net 1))
 (segment (start 121.8311 109.3236) (end 121.8311 111.2286) (width 0.4064) (layer "B.Cu") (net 1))
 (segment (start 134.0231 98.0206) (end 130.9751 101.0686) (width 0.3048) (layer "B.Cu") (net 1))
 (segment (start 135.6741 96.3696) (end 137.9601 96.3696) (width 0.3048) (layer "B.Cu") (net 1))
 (segment (start 164.3761 109.3236) (end 154.2161 109.3236) (width 0.4064) (layer "B.Cu") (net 1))
 (segment (start 166.2811 111.2286) (end 164.3761 109.3236) (width 0.4064) (layer "B.Cu") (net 1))
 (segment (start 152.3111 111.2286) (end 154.2161 109.3236) (width 0.4064) (layer "B.Cu") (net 1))
 (segment (start 137.0711 111.2286) (end 138.9761 109.3236) (width 0.4064) (layer "B.Cu") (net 1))
 (segment (start 120.5611 108.0536) (end 121.8311 109.3236) (width 0.4064) (layer "B.Cu") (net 1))
 (segment (start 154.2161 109.3236) (end 138.9761 109.3236) (width 0.4064) (layer "B.Cu") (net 1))
 (segment (start 138.9761 109.3236) (end 121.8311 109.3236) (width 0.4064) (layer "B.Cu") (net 1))
 (segment (start 130.9751 101.0686) (end 120.6881 101.0686) (width 0.3048) (layer "B.Cu") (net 1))
 (segment (start 134.0231 98.0206) (end 135.6741 96.3696) (width 0.3048) (layer "B.Cu") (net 1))
 (segment (start 120.5611 101.0686) (end 120.5611 108.0536) (width 0.4064) (layer "B.Cu") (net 1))
 (segment (start 136.6901 94.2106) (end 136.6901 86.9716) (width 0.3048) (layer "F.Cu") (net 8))
 (segment (start 131.4831 95.0996) (end 131.1021 94.7186) (width 0.3048) (layer "F.Cu") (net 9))
 (segment (start 131.1021 91.6706) (end 135.2931 87.4796) (width 0.3048) (layer "F.Cu") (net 9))
 (segment (start 132.2451 95.0996) (end 131.4831 95.0996) (width 0.3048) (layer "F.Cu") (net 9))
 (segment (start 131.1021 94.7186) (end 131.1021 91.6706) (width 0.3048) (layer "F.Cu") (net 9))
 (segment (start 120.6881 95.9886) (end 124.8791 100.1796) (width 0.3048) (layer "F.Cu") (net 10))
 (segment (start 124.8791 100.1796) (end 132.3721 100.1796) (width 0.3048) (layer "F.Cu") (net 10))
 (segment (start 126.7841 99.6716) (end 120.5611 93.4486) (width 0.3048) (layer "F.Cu") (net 7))
 (segment (start 132.2451 99.6716) (end 126.7841 99.6716) (width 0.3048) (layer "F.Cu") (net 7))
 (segment (start 132.3721 97.1316) (end 135.5471 97.1316) (width 0.3048) (layer "F.Cu") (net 6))
 (segment (start 136.0551 97.6396) (end 135.5471 97.1316) (width 0.3048) (layer "F.Cu") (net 6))
 (segment (start 132.3721 96.6236) (end 127.9271 96.6236) (width 0.3048) (layer "F.Cu") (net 6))
 (segment (start 134.1501 102.0846) (end 134.1501 99.5446) (width 0.3048) (layer "F.Cu") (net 6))
 (segment (start 134.1501 99.5446) (end 136.0551 97.6396) (width 0.3048) (layer "F.Cu") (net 6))
 (segment (start 132.3721 96.6236) (end 132.3721 97.1316) (width 0.3048) (layer "F.Cu") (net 6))
 (segment (start 140.3731 97.6396) (end 136.0551 97.6396) (width 0.3048) (layer "F.Cu") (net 6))
 (via (at 127.8001 96.6236) (size 0.7564) (drill 0.35) (layers "F.Cu" "B.Cu") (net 6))
 (segment (start 125.8951 98.5286) (end 120.5611 98.5286) (width 0.3048) (layer "B.Cu") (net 6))
 (segment (start 118.6561 100.4336) (end 118.6561 118.8486) (width 0.4064) (layer "B.Cu") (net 6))
 (segment (start 127.8001 96.6236) (end 125.8951 98.5286) (width 0.3048) (layer "B.Cu") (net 6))
 (segment (start 120.5611 98.5286) (end 118.6561 100.4336) (width 0.4064) (layer "B.Cu") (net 6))
 (segment (start 118.6561 118.8486) (end 173.9011 118.8486) (width 0.4064) (layer "B.Cu") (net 6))
 (segment (start 137.8331 106.1486) (end 142.0241 106.1486) (width 0.3048) (layer "F.Cu") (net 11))
 (segment (start 136.6901 102.4656) (end 136.6901 105.0056) (width 0.3048) (layer "F.Cu") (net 11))
 (segment (start 136.6901 105.0056) (end 137.8331 106.1486) (width 0.3048) (layer "F.Cu") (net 11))
 (segment (start 143.6751 104.4976) (end 144.5641 105.3866) (width 0.3048) (layer "F.Cu") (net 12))
 (segment (start 137.1981 102.4656) (end 137.1981 103.9896) (width 0.3048) (layer "F.Cu") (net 12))
 (segment (start 137.1981 103.9896) (end 137.7061 104.4976) (width 0.3048) (layer "F.Cu") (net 12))
 (segment (start 144.5641 105.3866) (end 144.5641 106.2756) (width 0.3048) (layer "F.Cu") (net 12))
 (segment (start 137.7061 104.4976) (end 143.6751 104.4976) (width 0.3048) (layer "F.Cu") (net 12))
 (segment (start 137.7061 102.3386) (end 137.7061 103.7356) (width 0.3048) (layer "F.Cu") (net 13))
 (segment (start 146.4691 103.9896) (end 147.2311 104.7516) (width 0.3048) (layer "F.Cu") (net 13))
 (segment (start 137.9601 103.9896) (end 146.4691 103.9896) (width 0.3048) (layer "F.Cu") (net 13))
 (segment (start 147.2311 104.7516) (end 147.2311 106.2756) (width 0.3048) (layer "F.Cu") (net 13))
 (segment (start 137.7061 103.7356) (end 137.9601 103.9896) (width 0.3048) (layer "F.Cu") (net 13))
 (segment (start 138.2141 103.3546) (end 138.3411 103.4816) (width 0.3048) (layer "F.Cu") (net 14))
 (segment (start 138.2141 102.3386) (end 138.2141 103.3546) (width 0.3048) (layer "F.Cu") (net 14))
 (segment (start 149.7711 104.4976) (end 149.7711 106.2756) (width 0.3048) (layer "F.Cu") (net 14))
 (segment (start 138.3411 103.4816) (end 148.7551 103.4816) (width 0.3048) (layer "F.Cu") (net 14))
 (segment (start 148.7551 103.4816) (end 149.7711 104.4976) (width 0.3048) (layer "F.Cu") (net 14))
 (segment (start 152.3111 104.8786) (end 152.3111 106.2756) (width 0.3048) (layer "F.Cu") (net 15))
 (segment (start 138.7221 102.4656) (end 138.7221 102.9736) (width 0.3048) (layer "F.Cu") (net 15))
 (segment (start 150.4061 102.9736) (end 152.3111 104.8786) (width 0.3048) (layer "F.Cu") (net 15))
 (segment (start 138.7221 102.9736) (end 150.4061 102.9736) (width 0.3048) (layer "F.Cu") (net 15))
 (segment (start 153.0731 102.4656) (end 154.8511 104.2436) (width 0.3048) (layer "F.Cu") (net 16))
 (segment (start 139.2301 102.4656) (end 153.0731 102.4656) (width 0.3048) (layer "F.Cu") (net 16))
 (segment (start 154.8511 104.2436) (end 154.8511 106.0216) (width 0.3048) (layer "F.Cu") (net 16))
 (segment (start 154.3431 100.6876) (end 154.8511 100.1796) (width 0.3048) (layer "F.Cu") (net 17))
 (segment (start 140.7541 100.6876) (end 154.3431 100.6876) (width 0.3048) (layer "F.Cu") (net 17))
 (segment (start 154.8511 100.1796) (end 154.8511 91.0356) (width 0.3048) (layer "F.Cu") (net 17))
 (segment (start 152.3111 98.9096) (end 152.3111 90.9086) (width 0.3048) (layer "F.Cu") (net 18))
 (segment (start 140.8811 100.1796) (end 151.0411 100.1796) (width 0.3048) (layer "F.Cu") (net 18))
 (segment (start 151.0411 100.1796) (end 152.3111 98.9096) (width 0.3048) (layer "F.Cu") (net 18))
 (segment (start 140.8811 99.6716) (end 148.8821 99.6716) (width 0.3048) (layer "F.Cu") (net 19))
 (segment (start 148.8821 99.6716) (end 149.7711 98.7826) (width 0.3048) (layer "F.Cu") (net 19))
 (segment (start 149.7711 98.7826) (end 149.7711 90.9086) (width 0.3048) (layer "F.Cu") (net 19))
 (segment (start 146.4691 99.1636) (end 147.2311 98.4016) (width 0.3048) (layer "F.Cu") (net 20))
 (segment (start 147.2311 98.4016) (end 147.2311 91.0356) (width 0.3048) (layer "F.Cu") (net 20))
 (segment (start 140.7541 99.1636) (end 146.4691 99.1636) (width 0.3048) (layer "F.Cu") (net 20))
 (segment (start 143.8021 98.6556) (end 144.6911 97.7666) (width 0.3048) (layer "F.Cu") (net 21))
 (segment (start 140.7541 98.6556) (end 143.8021 98.6556) (width 0.3048) (layer "F.Cu") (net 21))
 (segment (start 144.6911 97.7666) (end 144.6911 90.9086) (width 0.3048) (layer "F.Cu") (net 21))
 (segment (start 142.1511 97.6396) (end 142.1511 91.0356) (width 0.3048) (layer "F.Cu") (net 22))
 (segment (start 141.6431 98.1476) (end 142.1511 97.6396) (width 0.3048) (layer "F.Cu") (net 22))
 (segment (start 140.7541 98.1476) (end 141.6431 98.1476) (width 0.3048) (layer "F.Cu") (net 22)))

